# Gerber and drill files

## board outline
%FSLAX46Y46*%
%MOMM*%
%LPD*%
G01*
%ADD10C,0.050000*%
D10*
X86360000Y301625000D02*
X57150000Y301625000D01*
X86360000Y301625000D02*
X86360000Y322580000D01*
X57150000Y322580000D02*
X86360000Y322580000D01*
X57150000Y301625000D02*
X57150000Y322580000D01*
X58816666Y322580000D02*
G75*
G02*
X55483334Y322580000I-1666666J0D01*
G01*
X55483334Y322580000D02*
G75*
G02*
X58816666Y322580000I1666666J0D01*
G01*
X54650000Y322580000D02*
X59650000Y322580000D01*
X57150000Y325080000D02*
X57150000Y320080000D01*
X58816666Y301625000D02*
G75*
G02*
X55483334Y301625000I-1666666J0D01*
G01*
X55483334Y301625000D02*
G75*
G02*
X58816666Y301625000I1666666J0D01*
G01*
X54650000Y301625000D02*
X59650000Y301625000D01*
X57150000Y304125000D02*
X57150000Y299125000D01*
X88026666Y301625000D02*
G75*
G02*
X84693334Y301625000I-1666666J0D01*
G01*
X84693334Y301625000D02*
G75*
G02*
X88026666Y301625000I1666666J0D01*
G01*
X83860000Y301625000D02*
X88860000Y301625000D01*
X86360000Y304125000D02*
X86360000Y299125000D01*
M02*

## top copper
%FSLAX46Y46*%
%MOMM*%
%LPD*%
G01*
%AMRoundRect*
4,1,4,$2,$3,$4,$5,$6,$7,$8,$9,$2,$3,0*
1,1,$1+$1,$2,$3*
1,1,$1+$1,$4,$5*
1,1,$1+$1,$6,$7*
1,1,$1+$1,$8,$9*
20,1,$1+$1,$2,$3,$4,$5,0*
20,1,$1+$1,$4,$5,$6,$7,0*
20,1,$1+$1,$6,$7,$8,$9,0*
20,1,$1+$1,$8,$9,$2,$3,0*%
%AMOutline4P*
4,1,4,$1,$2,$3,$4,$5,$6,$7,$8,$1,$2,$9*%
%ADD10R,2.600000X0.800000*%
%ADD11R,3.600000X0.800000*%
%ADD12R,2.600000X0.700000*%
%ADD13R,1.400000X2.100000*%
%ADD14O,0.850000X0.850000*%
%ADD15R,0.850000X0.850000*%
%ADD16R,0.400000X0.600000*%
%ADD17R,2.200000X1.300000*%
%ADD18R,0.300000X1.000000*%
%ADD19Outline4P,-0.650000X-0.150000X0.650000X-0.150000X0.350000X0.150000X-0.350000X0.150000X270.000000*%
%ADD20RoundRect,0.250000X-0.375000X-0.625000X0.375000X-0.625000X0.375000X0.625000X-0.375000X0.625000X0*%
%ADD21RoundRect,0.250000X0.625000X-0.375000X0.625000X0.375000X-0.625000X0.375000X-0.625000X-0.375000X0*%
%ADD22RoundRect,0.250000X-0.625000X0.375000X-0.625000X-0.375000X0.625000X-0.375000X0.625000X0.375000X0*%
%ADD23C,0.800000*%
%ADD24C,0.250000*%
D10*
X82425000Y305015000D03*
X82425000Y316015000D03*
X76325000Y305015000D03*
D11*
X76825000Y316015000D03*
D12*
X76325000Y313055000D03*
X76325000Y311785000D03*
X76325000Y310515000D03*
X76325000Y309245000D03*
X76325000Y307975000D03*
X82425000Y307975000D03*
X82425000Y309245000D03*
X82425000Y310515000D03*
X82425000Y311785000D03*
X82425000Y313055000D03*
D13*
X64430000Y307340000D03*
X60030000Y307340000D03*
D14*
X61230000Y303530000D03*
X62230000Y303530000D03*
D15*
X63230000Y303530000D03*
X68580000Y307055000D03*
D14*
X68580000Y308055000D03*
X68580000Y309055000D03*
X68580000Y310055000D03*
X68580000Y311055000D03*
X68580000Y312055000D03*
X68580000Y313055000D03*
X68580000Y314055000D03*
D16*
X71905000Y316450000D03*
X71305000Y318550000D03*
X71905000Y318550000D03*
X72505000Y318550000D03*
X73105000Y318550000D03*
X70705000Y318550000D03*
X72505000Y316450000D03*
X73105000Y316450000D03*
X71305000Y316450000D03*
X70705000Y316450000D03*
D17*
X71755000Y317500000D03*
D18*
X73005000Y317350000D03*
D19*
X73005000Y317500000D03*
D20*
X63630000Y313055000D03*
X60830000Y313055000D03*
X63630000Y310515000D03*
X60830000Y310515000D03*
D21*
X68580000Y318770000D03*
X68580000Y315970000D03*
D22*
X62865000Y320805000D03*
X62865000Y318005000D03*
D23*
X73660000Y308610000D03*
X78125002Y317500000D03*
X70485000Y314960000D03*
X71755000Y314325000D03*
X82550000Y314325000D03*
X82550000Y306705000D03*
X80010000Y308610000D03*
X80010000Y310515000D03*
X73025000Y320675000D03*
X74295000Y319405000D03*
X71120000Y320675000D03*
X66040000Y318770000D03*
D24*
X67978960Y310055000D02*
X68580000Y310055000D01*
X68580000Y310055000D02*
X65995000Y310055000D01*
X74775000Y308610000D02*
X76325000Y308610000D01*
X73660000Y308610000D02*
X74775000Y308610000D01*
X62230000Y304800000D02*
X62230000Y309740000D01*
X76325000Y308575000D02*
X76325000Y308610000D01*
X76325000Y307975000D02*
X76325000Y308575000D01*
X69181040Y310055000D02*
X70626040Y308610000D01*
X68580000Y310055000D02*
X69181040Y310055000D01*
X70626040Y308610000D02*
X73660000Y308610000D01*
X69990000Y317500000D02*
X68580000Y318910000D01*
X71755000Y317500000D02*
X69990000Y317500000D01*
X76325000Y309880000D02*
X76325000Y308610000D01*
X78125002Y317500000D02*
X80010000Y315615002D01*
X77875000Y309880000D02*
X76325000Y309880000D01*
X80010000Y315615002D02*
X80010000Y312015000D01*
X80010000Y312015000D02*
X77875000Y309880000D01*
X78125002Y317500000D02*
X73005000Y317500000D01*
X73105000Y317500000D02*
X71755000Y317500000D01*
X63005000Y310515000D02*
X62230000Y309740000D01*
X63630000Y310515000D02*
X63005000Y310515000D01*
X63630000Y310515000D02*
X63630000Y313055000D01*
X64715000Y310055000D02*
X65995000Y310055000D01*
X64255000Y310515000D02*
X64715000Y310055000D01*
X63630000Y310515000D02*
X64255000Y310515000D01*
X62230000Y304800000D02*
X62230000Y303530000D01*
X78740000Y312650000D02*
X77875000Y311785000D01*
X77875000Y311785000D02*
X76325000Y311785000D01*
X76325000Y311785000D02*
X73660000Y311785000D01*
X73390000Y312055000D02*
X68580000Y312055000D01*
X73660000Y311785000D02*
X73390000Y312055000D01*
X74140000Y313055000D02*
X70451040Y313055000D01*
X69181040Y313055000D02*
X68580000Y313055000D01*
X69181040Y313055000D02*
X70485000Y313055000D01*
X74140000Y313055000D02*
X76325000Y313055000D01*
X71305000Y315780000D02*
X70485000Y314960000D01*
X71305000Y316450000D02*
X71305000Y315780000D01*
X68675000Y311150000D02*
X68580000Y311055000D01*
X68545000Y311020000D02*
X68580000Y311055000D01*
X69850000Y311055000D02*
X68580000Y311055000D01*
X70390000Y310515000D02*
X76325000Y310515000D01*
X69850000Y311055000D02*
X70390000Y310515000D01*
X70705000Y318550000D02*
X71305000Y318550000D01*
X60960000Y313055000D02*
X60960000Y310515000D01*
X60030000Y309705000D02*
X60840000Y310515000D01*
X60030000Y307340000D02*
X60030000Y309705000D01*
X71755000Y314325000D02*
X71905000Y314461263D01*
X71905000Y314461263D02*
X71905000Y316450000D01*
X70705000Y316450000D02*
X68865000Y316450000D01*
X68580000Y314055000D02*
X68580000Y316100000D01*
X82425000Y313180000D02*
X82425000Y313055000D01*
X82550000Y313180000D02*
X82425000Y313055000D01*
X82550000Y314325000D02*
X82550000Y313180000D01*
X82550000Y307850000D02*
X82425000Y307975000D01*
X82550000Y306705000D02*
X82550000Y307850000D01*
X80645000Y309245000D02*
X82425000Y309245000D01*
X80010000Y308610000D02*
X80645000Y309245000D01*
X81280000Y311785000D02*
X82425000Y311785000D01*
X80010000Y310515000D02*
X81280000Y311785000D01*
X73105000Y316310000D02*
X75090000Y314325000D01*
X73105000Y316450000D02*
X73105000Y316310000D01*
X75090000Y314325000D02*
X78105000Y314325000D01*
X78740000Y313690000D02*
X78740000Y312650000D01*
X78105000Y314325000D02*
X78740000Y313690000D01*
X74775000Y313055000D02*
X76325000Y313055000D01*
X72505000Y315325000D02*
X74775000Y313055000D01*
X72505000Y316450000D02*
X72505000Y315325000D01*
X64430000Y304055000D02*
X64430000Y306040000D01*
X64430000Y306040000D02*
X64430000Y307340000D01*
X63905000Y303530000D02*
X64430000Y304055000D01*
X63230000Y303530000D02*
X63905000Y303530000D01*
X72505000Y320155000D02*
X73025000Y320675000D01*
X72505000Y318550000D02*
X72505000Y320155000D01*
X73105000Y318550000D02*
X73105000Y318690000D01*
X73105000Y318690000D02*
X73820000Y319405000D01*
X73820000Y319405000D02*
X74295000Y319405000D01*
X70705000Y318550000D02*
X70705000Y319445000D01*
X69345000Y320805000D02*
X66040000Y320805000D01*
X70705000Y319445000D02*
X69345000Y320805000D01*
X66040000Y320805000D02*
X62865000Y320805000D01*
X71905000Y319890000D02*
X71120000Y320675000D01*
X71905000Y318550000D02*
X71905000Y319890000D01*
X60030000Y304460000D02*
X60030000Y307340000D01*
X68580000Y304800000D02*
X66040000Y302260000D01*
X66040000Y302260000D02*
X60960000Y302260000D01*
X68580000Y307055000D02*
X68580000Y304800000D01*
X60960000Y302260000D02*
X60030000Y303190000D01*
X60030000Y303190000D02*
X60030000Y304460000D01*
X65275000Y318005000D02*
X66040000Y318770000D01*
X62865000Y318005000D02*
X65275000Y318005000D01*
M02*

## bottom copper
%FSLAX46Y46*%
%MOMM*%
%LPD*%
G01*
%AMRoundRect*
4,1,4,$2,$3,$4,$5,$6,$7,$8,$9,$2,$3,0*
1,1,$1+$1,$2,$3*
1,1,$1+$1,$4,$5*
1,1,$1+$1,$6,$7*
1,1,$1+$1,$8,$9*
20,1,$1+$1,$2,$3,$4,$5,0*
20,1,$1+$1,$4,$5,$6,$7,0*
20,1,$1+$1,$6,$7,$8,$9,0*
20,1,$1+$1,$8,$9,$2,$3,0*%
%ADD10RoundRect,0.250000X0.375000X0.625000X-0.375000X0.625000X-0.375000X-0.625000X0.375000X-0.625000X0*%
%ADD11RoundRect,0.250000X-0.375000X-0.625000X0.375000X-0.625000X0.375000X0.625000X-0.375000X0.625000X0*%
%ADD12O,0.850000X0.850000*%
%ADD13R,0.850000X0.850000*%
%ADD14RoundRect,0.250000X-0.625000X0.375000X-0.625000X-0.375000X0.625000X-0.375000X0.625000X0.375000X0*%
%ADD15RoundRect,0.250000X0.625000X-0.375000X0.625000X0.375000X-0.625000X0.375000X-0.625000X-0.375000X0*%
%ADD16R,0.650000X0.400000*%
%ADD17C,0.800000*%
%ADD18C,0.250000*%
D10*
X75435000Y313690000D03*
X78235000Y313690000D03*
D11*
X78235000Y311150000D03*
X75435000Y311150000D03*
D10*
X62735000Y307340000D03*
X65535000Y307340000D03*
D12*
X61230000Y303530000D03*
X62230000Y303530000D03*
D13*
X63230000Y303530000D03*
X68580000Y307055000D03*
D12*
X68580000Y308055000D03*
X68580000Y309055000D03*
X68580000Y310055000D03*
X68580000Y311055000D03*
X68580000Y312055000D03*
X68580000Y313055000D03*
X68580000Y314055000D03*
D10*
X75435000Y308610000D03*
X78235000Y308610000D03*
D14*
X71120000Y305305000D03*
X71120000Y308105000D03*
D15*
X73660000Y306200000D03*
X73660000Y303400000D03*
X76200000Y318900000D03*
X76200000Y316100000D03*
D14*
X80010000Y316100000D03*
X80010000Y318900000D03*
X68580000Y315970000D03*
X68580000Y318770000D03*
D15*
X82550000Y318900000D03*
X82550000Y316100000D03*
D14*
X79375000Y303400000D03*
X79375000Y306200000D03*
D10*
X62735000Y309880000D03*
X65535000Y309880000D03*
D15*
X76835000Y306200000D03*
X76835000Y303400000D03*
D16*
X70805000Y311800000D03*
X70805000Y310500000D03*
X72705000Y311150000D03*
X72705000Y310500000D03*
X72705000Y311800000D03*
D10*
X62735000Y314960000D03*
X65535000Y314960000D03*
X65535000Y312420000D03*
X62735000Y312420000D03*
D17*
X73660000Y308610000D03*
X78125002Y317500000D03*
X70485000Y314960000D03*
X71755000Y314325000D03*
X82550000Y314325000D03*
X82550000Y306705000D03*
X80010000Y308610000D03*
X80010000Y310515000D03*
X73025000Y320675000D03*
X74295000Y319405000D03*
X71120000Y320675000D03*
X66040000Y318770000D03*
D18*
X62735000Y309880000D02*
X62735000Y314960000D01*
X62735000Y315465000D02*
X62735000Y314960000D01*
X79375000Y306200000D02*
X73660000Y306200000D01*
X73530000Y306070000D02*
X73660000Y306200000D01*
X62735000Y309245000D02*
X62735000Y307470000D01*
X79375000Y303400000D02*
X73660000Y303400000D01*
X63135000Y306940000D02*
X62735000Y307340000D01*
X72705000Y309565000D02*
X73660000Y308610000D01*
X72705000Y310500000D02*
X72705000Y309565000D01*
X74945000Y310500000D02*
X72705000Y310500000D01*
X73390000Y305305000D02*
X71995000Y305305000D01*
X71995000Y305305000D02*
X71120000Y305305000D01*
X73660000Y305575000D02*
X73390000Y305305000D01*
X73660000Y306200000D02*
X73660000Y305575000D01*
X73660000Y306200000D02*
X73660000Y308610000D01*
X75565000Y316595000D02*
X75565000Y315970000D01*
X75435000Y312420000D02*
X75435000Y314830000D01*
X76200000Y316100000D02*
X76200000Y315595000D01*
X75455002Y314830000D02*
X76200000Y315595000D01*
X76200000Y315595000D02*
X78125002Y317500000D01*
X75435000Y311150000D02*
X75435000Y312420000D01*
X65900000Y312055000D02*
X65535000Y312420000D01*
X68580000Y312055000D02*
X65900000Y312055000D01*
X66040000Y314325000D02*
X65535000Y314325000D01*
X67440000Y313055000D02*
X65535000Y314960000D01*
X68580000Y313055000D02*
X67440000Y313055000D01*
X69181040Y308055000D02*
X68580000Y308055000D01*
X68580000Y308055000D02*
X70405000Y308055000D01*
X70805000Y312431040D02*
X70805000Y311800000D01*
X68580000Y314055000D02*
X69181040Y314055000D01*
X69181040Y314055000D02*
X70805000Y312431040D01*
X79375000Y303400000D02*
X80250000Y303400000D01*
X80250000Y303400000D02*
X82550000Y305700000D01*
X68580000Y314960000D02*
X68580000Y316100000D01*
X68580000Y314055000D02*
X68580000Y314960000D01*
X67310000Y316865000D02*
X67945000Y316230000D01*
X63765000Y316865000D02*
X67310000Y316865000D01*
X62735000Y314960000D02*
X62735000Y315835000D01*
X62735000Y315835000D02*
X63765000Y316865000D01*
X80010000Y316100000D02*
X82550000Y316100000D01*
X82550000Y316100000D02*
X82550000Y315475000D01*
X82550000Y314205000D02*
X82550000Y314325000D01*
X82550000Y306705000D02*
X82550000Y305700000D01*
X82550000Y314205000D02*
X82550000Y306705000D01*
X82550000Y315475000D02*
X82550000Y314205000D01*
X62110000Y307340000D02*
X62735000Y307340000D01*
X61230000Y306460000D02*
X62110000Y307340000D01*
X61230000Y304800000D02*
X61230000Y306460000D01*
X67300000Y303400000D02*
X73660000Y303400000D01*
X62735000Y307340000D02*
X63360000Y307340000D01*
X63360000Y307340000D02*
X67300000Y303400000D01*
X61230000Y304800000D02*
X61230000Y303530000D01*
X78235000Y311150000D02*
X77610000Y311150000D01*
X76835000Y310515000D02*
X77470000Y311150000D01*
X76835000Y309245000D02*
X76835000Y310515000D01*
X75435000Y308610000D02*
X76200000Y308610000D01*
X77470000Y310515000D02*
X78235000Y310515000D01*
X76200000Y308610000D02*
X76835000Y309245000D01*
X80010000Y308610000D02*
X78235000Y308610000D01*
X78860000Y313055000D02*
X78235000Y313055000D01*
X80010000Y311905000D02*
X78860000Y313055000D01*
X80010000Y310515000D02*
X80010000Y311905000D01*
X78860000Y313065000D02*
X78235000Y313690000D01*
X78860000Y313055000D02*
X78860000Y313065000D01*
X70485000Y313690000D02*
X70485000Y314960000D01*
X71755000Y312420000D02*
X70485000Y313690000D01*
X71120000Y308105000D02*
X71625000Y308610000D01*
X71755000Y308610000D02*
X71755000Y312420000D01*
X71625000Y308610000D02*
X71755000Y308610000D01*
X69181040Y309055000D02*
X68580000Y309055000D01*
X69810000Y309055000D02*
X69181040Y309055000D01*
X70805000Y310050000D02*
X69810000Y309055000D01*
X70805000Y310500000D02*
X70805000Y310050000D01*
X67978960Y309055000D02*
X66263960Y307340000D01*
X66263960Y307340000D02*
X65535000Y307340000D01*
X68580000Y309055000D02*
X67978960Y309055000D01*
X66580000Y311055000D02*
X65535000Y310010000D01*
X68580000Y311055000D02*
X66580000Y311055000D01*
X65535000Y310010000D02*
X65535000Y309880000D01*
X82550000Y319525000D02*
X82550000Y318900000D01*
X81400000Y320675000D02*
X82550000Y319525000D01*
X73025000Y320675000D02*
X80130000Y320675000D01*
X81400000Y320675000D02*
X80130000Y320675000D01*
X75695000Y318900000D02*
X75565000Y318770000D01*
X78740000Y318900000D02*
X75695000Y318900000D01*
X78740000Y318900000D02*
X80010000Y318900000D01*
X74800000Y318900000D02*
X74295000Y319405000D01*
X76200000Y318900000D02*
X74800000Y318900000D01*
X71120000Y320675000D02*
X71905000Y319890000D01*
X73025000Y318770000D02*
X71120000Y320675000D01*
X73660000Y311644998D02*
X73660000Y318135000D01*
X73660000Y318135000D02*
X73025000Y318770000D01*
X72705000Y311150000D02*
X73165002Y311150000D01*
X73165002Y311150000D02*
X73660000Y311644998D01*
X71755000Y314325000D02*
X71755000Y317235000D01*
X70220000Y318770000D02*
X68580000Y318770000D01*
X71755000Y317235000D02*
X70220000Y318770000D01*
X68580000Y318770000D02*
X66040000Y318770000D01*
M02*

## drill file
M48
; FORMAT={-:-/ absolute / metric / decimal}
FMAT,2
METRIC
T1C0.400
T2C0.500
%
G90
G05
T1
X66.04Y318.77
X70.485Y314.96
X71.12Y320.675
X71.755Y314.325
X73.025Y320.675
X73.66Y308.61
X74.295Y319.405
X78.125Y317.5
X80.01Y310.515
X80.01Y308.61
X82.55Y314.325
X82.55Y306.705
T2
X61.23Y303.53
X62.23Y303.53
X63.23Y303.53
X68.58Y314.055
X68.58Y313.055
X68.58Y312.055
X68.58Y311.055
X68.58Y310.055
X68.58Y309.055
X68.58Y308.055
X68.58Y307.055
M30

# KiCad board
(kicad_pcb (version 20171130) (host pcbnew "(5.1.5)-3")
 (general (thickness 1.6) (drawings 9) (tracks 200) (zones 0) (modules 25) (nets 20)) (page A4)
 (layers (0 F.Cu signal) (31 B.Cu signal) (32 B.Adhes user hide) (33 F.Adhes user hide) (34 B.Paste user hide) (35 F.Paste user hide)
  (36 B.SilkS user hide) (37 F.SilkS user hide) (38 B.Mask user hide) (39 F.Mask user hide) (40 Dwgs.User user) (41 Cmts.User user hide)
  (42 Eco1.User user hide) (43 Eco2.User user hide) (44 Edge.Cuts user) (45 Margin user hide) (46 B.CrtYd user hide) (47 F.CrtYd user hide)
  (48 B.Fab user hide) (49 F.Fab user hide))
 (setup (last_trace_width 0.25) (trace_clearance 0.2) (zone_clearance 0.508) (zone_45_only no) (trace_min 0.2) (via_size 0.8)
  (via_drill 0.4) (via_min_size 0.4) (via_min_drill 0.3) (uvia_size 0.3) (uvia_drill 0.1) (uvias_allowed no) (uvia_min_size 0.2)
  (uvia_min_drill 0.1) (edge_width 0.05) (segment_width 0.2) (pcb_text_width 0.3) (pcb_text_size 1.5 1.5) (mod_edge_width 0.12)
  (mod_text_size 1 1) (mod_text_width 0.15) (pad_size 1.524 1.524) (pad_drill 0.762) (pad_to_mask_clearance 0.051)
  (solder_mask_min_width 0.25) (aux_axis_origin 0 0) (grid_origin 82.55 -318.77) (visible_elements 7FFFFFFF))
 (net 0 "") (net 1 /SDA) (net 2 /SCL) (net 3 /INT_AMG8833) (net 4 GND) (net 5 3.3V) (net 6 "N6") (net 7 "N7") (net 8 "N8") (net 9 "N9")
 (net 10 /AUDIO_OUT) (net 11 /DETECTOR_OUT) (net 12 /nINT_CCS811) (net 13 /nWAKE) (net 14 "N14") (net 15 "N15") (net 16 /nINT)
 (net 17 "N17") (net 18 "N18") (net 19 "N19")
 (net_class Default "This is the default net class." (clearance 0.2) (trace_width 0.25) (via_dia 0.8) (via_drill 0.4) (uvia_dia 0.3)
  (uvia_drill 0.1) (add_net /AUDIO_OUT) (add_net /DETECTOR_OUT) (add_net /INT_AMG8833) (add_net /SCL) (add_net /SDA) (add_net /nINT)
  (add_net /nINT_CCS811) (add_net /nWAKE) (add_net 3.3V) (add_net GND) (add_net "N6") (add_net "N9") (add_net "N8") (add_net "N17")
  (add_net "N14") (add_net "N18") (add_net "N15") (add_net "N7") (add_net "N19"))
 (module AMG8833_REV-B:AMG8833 (layer F.Cu) (at 79.375 -310.515 270)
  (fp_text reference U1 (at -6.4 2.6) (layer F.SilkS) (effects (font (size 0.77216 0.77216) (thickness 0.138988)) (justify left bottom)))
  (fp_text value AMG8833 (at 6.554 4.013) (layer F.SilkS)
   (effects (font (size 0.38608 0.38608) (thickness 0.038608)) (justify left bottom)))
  (pad 8 smd rect (at 5.5 -3.05) (size 2.6 0.8) (layers F.Cu F.Paste F.Mask) (solder_mask_margin 0.0508))
  (pad 14 smd rect (at -5.5 -3.05) (size 2.6 0.8) (layers F.Cu F.Paste F.Mask) (solder_mask_margin 0.0508))
  (pad 7 smd rect (at 5.5 3.05) (size 2.6 0.8) (layers F.Cu F.Paste F.Mask) (solder_mask_margin 0.0508))
  (pad 1 smd rect (at -5.5 2.55) (size 3.6 0.8) (layers F.Cu F.Paste F.Mask) (solder_mask_margin 0.0508))
  (pad 2 smd rect (at -2.54 3.05) (size 2.6 0.7) (layers F.Cu F.Paste F.Mask) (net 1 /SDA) (solder_mask_margin 0.0508))
  (pad 3 smd rect (at -1.27 3.05) (size 2.6 0.7) (layers F.Cu F.Paste F.Mask) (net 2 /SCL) (solder_mask_margin 0.0508))
  (pad 4 smd rect (at 0 3.05) (size 2.6 0.7) (layers F.Cu F.Paste F.Mask) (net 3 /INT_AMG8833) (solder_mask_margin 0.0508))
  (pad 5 smd rect (at 1.27 3.05) (size 2.6 0.7) (layers F.Cu F.Paste F.Mask) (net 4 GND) (solder_mask_margin 0.0508))
  (pad 6 smd rect (at 2.54 3.05) (size 2.6 0.7) (layers F.Cu F.Paste F.Mask) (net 4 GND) (solder_mask_margin 0.0508))
  (pad 9 smd rect (at 2.54 -3.05) (size 2.6 0.7) (layers F.Cu F.Paste F.Mask) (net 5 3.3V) (solder_mask_margin 0.0508))
  (pad 10 smd rect (at 1.27 -3.05) (size 2.6 0.7) (layers F.Cu F.Paste F.Mask) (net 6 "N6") (solder_mask_margin 0.0508))
  (pad 11 smd rect (at 0 -3.05) (size 2.6 0.7) (layers F.Cu F.Paste F.Mask) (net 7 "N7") (solder_mask_margin 0.0508))
  (pad 12 smd rect (at -1.27 -3.05) (size 2.6 0.7) (layers F.Cu F.Paste F.Mask) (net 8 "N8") (solder_mask_margin 0.0508))
  (pad 13 smd rect (at -2.54 -3.05) (size 2.6 0.7) (layers F.Cu F.Paste F.Mask) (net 5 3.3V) (solder_mask_margin 0.0508)))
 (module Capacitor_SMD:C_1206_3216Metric (layer B.Cu) (at 76.835 -313.69 180)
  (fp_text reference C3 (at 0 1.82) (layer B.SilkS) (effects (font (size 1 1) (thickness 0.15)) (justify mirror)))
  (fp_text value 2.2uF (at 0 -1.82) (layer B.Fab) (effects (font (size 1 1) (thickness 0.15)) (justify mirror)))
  (pad 2 smd roundrect (at 1.4 0 180) (size 1.25 1.75) (layers B.Cu B.Paste B.Mask) (roundrect_rratio 0.2) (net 4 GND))
  (pad 1 smd roundrect (at -1.4 0 180) (size 1.25 1.75) (layers B.Cu B.Paste B.Mask) (roundrect_rratio 0.2) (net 8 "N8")))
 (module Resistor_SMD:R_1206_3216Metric (layer B.Cu) (at 76.835 -311.15)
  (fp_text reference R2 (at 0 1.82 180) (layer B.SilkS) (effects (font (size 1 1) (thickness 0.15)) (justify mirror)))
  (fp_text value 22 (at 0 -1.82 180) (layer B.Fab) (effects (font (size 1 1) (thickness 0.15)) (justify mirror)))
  (pad 2 smd roundrect (at 1.4 0) (size 1.25 1.75) (layers B.Cu B.Paste B.Mask) (roundrect_rratio 0.2) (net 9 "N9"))
  (pad 1 smd roundrect (at -1.4 0) (size 1.25 1.75) (layers B.Cu B.Paste B.Mask) (roundrect_rratio 0.2) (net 4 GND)))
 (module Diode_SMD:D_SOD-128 (layer F.Cu) (at 62.23 -307.34)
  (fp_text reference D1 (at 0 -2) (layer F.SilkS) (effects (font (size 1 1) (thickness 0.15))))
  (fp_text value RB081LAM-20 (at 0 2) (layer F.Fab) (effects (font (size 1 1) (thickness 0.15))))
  (pad 2 smd rect (at 2.2 0) (size 1.4 2.1) (layers F.Cu F.Paste F.Mask) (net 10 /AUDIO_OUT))
  (pad 1 smd rect (at -2.2 0) (size 1.4 2.1) (layers F.Cu F.Paste F.Mask) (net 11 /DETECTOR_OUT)))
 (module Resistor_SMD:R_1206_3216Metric (layer B.Cu) (at 64.135 -307.34 180)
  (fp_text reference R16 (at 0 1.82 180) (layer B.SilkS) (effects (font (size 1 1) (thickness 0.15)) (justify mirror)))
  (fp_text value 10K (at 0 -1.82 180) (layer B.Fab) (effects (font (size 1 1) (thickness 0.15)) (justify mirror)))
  (pad 2 smd roundrect (at 1.4 0 180) (size 1.25 1.75) (layers B.Cu B.Paste B.Mask) (roundrect_rratio 0.2) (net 5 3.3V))
  (pad 1 smd roundrect (at -1.4 0 180) (size 1.25 1.75) (layers B.Cu B.Paste B.Mask) (roundrect_rratio 0.2) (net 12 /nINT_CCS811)))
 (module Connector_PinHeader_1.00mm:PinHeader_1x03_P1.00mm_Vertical (layer F.Cu) (at 63.23 -303.53 270)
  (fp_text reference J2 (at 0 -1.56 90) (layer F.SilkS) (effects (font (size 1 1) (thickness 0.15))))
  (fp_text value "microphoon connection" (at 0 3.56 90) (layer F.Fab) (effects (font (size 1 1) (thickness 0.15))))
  (pad 3 thru_hole oval (at 0 2 270) (size 0.85 0.85) (drill 0.5) (layers *.Cu *.Mask) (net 5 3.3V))
  (pad 2 thru_hole oval (at 0 1 270) (size 0.85 0.85) (drill 0.5) (layers *.Cu *.Mask) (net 4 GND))
  (pad 1 thru_hole rect (at 0 0 270) (size 0.85 0.85) (drill 0.5) (layers *.Cu *.Mask) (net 10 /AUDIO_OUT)))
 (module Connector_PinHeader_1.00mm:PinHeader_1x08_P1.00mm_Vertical (layer F.Cu) (at 68.58 -307.055 180)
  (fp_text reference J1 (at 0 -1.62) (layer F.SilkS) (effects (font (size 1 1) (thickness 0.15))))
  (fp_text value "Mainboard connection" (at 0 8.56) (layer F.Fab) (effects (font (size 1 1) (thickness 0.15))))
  (pad 1 thru_hole rect (at 0 0 180) (size 0.85 0.85) (drill 0.5) (layers *.Cu *.Mask) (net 11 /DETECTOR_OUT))
  (pad 2 thru_hole oval (at 0 1 180) (size 0.85 0.85) (drill 0.5) (layers *.Cu *.Mask) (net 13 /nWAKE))
  (pad 3 thru_hole oval (at 0 2 180) (size 0.85 0.85) (drill 0.5) (layers *.Cu *.Mask) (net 12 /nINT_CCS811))
  (pad 4 thru_hole oval (at 0 3 180) (size 0.85 0.85) (drill 0.5) (layers *.Cu *.Mask) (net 4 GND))
  (pad 5 thru_hole oval (at 0 4 180) (size 0.85 0.85) (drill 0.5) (layers *.Cu *.Mask) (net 3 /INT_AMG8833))
  (pad 6 thru_hole oval (at 0 5 180) (size 0.85 0.85) (drill 0.5) (layers *.Cu *.Mask) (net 2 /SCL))
  (pad 7 thru_hole oval (at 0 6 180) (size 0.85 0.85) (drill 0.5) (layers *.Cu *.Mask) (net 1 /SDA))
  (pad 8 thru_hole oval (at 0 7 180) (size 0.85 0.85) (drill 0.5) (layers *.Cu *.Mask) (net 5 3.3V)))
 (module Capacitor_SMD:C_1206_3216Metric (layer B.Cu) (at 76.835 -308.61 180)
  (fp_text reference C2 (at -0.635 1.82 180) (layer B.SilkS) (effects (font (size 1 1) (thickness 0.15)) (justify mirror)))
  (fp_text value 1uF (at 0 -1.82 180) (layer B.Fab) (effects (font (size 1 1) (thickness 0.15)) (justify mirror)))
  (pad 2 smd roundrect (at 1.4 0 180) (size 1.25 1.75) (layers B.Cu B.Paste B.Mask) (roundrect_rratio 0.2) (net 9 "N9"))
  (pad 1 smd roundrect (at -1.4 0 180) (size 1.25 1.75) (layers B.Cu B.Paste B.Mask) (roundrect_rratio 0.2) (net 6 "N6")))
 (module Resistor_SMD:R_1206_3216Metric (layer B.Cu) (at 71.12 -306.705 270)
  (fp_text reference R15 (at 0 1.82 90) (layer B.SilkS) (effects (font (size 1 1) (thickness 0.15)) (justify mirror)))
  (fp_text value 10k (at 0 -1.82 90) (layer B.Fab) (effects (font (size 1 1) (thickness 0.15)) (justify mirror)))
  (pad 2 smd roundrect (at 1.4 0 270) (size 1.25 1.75) (layers B.Cu B.Paste B.Mask) (roundrect_rratio 0.2) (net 4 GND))
  (pad 1 smd roundrect (at -1.4 0 270) (size 1.25 1.75) (layers B.Cu B.Paste B.Mask) (roundrect_rratio 0.2) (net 13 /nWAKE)))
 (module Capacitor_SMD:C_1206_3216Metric (layer B.Cu) (at 73.66 -304.8 90)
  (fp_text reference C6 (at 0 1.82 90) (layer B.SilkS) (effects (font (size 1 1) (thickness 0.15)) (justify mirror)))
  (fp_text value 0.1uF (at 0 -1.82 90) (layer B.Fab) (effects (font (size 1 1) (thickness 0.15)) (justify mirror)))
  (pad 2 smd roundrect (at 1.4 0 90) (size 1.25 1.75) (layers B.Cu B.Paste B.Mask) (roundrect_rratio 0.2) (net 4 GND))
  (pad 1 smd roundrect (at -1.4 0 90) (size 1.25 1.75) (layers B.Cu B.Paste B.Mask) (roundrect_rratio 0.2) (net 5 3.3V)))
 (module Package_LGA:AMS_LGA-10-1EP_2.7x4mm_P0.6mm (layer F.Cu) (at 71.905 -317.5 270)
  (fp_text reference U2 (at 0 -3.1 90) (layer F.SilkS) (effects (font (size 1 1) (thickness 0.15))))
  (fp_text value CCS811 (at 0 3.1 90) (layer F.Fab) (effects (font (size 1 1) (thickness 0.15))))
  (pad 8 smd rect (at 1.05 0 270) (size 0.6 0.4) (layers F.Cu F.Paste F.Mask) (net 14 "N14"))
  (pad 4 smd rect (at -1.05 0.6 270) (size 0.6 0.4) (layers F.Cu F.Paste F.Mask) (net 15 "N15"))
  (pad 3 smd rect (at -1.05 0 270) (size 0.6 0.4) (layers F.Cu F.Paste F.Mask) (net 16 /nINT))
  (pad 2 smd rect (at -1.05 -0.6 270) (size 0.6 0.4) (layers F.Cu F.Paste F.Mask) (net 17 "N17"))
  (pad 1 smd rect (at -1.05 -1.2 270) (size 0.6 0.4) (layers F.Cu F.Paste F.Mask) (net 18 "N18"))
  (pad 5 smd rect (at -1.05 1.2 270) (size 0.6 0.4) (layers F.Cu F.Paste F.Mask) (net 15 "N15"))
  (pad 9 smd rect (at 1.05 -0.6 270) (size 0.6 0.4) (layers F.Cu F.Paste F.Mask) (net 1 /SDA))
  (pad 10 smd rect (at 1.05 -1.2 270) (size 0.6 0.4) (layers F.Cu F.Paste F.Mask) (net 2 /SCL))
  (pad 7 smd rect (at 1.05 0.6 270) (size 0.6 0.4) (layers F.Cu F.Paste F.Mask) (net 13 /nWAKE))
  (pad 6 smd rect (at 1.05 1.2 270) (size 0.6 0.4) (layers F.Cu F.Paste F.Mask) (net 5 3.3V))
  (pad 11 smd rect (at 0 0.15 270) (size 1.3 2.2) (layers F.Cu F.Paste F.Mask) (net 4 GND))
  (pad 11 smd rect (at 0.15 -1.1 270) (size 1 0.3) (layers F.Cu F.Paste F.Mask) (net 4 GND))
  (pad 11 smd trapezoid (at 0 -1.1 270) (size 1 0.3) (rect_delta 0 0.3) (layers F.Cu F.Paste F.Mask) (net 4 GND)))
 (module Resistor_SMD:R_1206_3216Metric (layer F.Cu) (at 62.23 -313.055)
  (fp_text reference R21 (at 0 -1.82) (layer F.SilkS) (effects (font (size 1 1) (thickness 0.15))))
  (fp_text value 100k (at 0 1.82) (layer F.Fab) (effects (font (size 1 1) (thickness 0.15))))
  (pad 2 smd roundrect (at 1.4 0) (size 1.25 1.75) (layers F.Cu F.Paste F.Mask) (roundrect_rratio 0.2) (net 4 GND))
  (pad 1 smd roundrect (at -1.4 0) (size 1.25 1.75) (layers F.Cu F.Paste F.Mask) (roundrect_rratio 0.2) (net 11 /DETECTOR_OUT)))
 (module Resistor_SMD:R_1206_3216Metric (layer B.Cu) (at 76.2 -317.5 90)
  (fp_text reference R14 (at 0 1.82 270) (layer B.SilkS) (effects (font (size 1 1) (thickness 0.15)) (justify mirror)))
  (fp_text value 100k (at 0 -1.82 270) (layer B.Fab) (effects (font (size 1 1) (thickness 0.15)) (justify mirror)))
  (pad 2 smd roundrect (at 1.4 0 90) (size 1.25 1.75) (layers B.Cu B.Paste B.Mask) (roundrect_rratio 0.2) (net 18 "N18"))
  (pad 1 smd roundrect (at -1.4 0 90) (size 1.25 1.75) (layers B.Cu B.Paste B.Mask) (roundrect_rratio 0.2) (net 4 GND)))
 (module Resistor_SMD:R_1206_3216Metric (layer B.Cu) (at 80.01 -317.5 270)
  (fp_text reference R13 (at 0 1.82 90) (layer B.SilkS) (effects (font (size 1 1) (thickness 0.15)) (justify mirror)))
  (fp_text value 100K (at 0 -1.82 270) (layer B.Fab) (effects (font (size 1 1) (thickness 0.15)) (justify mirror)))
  (pad 2 smd roundrect (at 1.4 0 270) (size 1.25 1.75) (layers B.Cu B.Paste B.Mask) (roundrect_rratio 0.2) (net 5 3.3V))
  (pad 1 smd roundrect (at -1.4 0 270) (size 1.25 1.75) (layers B.Cu B.Paste B.Mask) (roundrect_rratio 0.2) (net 18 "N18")))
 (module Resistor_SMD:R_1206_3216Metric (layer B.Cu) (at 68.58 -317.37 270)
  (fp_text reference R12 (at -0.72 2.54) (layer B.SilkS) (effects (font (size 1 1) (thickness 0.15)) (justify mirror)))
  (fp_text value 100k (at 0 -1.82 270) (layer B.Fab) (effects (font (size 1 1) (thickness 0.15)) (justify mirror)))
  (pad 2 smd roundrect (at 1.4 0 270) (size 1.25 1.75) (layers B.Cu B.Paste B.Mask) (roundrect_rratio 0.2) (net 5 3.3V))
  (pad 1 smd roundrect (at -1.4 0 270) (size 1.25 1.75) (layers B.Cu B.Paste B.Mask) (roundrect_rratio 0.2) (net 14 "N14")))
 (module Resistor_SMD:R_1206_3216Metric (layer B.Cu) (at 82.55 -317.5 90)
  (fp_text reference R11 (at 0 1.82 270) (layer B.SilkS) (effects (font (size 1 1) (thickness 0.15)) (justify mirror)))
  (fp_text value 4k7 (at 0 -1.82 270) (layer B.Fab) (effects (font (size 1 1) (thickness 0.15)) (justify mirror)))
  (pad 2 smd roundrect (at 1.4 0 90) (size 1.25 1.75) (layers B.Cu B.Paste B.Mask) (roundrect_rratio 0.2) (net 17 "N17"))
  (pad 1 smd roundrect (at -1.4 0 90) (size 1.25 1.75) (layers B.Cu B.Paste B.Mask) (roundrect_rratio 0.2) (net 5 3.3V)))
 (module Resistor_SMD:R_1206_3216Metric (layer B.Cu) (at 79.375 -304.8 270)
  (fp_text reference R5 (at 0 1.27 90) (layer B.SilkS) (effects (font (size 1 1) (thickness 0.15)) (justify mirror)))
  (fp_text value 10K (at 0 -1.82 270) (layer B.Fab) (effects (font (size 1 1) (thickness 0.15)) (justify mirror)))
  (pad 2 smd roundrect (at 1.4 0 270) (size 1.25 1.75) (layers B.Cu B.Paste B.Mask) (roundrect_rratio 0.2) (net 5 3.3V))
  (pad 1 smd roundrect (at -1.4 0 270) (size 1.25 1.75) (layers B.Cu B.Paste B.Mask) (roundrect_rratio 0.2) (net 4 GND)))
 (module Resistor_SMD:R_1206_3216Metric (layer B.Cu) (at 64.135 -309.88 180)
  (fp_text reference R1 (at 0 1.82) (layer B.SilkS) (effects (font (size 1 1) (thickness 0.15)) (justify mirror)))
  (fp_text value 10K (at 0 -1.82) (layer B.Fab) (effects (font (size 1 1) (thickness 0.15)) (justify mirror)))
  (pad 2 smd roundrect (at 1.4 0 180) (size 1.25 1.75) (layers B.Cu B.Paste B.Mask) (roundrect_rratio 0.2) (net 5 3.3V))
  (pad 1 smd roundrect (at -1.4 0 180) (size 1.25 1.75) (layers B.Cu B.Paste B.Mask) (roundrect_rratio 0.2) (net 3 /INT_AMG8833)))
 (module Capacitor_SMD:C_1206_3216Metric (layer F.Cu) (at 62.23 -310.515)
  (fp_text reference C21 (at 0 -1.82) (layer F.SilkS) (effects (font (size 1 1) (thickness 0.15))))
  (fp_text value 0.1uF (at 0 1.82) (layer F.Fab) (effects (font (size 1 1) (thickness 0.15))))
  (pad 2 smd roundrect (at 1.4 0) (size 1.25 1.75) (layers F.Cu F.Paste F.Mask) (roundrect_rratio 0.2) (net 4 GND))
  (pad 1 smd roundrect (at -1.4 0) (size 1.25 1.75) (layers F.Cu F.Paste F.Mask) (roundrect_rratio 0.2) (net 11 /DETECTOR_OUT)))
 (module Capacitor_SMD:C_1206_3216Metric (layer F.Cu) (at 68.58 -317.37 90)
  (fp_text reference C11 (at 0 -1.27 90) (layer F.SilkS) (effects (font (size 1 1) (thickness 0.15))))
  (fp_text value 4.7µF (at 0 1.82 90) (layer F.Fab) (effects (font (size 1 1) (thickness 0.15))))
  (pad 2 smd roundrect (at 1.4 0 90) (size 1.25 1.75) (layers F.Cu F.Paste F.Mask) (roundrect_rratio 0.2) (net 4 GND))
  (pad 1 smd roundrect (at -1.4 0 90) (size 1.25 1.75) (layers F.Cu F.Paste F.Mask) (roundrect_rratio 0.2) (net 5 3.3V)))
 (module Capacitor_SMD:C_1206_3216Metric (layer B.Cu) (at 76.835 -304.8 90)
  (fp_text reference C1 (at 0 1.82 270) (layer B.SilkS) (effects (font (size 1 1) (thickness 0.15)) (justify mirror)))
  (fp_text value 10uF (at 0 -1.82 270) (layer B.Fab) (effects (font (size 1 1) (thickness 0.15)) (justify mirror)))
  (pad 2 smd roundrect (at 1.4 0 90) (size 1.25 1.75) (layers B.Cu B.Paste B.Mask) (roundrect_rratio 0.2) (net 4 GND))
  (pad 1 smd roundrect (at -1.4 0 90) (size 1.25 1.75) (layers B.Cu B.Paste B.Mask) (roundrect_rratio 0.2) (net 5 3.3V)))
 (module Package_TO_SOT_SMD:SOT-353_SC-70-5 (layer B.Cu) (at 71.755 -311.15 180)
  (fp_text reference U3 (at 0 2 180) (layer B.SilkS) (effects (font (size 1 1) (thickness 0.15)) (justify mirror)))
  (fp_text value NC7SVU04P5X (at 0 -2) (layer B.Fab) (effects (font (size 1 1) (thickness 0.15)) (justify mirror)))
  (pad 5 smd rect (at 0.95 0.65 180) (size 0.65 0.4) (layers B.Cu B.Paste B.Mask) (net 5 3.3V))
  (pad 4 smd rect (at 0.95 -0.65 180) (size 0.65 0.4) (layers B.Cu B.Paste B.Mask) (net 12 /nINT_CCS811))
  (pad 2 smd rect (at -0.95 0 180) (size 0.65 0.4) (layers B.Cu B.Paste B.Mask) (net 16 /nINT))
  (pad 3 smd rect (at -0.95 -0.65 180) (size 0.65 0.4) (layers B.Cu B.Paste B.Mask) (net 4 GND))
  (pad 1 smd rect (at -0.95 0.65 180) (size 0.65 0.4) (layers B.Cu B.Paste B.Mask) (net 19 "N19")))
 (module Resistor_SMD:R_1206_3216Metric (layer B.Cu) (at 64.135 -314.96 180)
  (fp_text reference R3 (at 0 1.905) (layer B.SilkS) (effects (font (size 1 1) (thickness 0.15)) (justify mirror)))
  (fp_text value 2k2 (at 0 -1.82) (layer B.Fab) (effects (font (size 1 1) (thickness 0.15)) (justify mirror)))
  (pad 2 smd roundrect (at 1.4 0 180) (size 1.25 1.75) (layers B.Cu B.Paste B.Mask) (roundrect_rratio 0.2) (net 5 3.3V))
  (pad 1 smd roundrect (at -1.4 0 180) (size 1.25 1.75) (layers B.Cu B.Paste B.Mask) (roundrect_rratio 0.2) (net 1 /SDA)))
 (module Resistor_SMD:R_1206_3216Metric (layer B.Cu) (at 64.135 -312.42 180)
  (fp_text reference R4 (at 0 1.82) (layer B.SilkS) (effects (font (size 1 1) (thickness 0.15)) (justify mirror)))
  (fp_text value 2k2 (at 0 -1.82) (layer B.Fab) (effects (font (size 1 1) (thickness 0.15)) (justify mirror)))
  (pad 1 smd roundrect (at -1.4 0 180) (size 1.25 1.75) (layers B.Cu B.Paste B.Mask) (roundrect_rratio 0.2) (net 2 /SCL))
  (pad 2 smd roundrect (at 1.4 0 180) (size 1.25 1.75) (layers B.Cu B.Paste B.Mask) (roundrect_rratio 0.2) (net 5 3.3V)))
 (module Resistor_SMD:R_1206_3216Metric (layer F.Cu) (at 62.865 -319.405 270)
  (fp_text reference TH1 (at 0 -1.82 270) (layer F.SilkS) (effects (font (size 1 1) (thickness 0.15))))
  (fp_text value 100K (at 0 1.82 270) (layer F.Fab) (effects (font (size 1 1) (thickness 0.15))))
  (pad 1 smd roundrect (at -1.4 0 270) (size 1.25 1.75) (layers F.Cu F.Paste F.Mask) (roundrect_rratio 0.2) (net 15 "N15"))
  (pad 2 smd roundrect (at 1.4 0 270) (size 1.25 1.75) (layers F.Cu F.Paste F.Mask) (roundrect_rratio 0.2) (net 14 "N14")))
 (gr_line (start 86.36 -301.625) (end 57.15 -301.625) (layer Edge.Cuts) (width 0.05))
 (gr_line (start 86.36 -301.625) (end 86.36 -322.58) (layer Edge.Cuts) (width 0.05))
 (gr_line (start 57.15 -322.58) (end 86.36 -322.58) (layer Edge.Cuts) (width 0.05))
 (gr_line (start 57.15 -301.625) (end 57.15 -322.58) (layer Edge.Cuts) (width 0.05))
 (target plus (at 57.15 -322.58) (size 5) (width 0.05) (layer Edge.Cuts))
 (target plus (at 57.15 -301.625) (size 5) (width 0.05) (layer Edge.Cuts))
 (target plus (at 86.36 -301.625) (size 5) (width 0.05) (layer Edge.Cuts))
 (segment (start 67.97896 -310.055) (end 68.58 -310.055) (width 0.25) (layer F.Cu) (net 4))
 (segment (start 62.735 -309.88) (end 62.735 -314.96) (width 0.25) (layer B.Cu) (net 5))
 (segment (start 62.735 -315.465) (end 62.735 -314.96) (width 0.25) (layer B.Cu) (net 5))
 (segment (start 79.375 -306.2) (end 73.66 -306.2) (width 0.25) (layer B.Cu) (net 4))
 (segment (start 68.58 -310.055) (end 65.995 -310.055) (width 0.25) (layer F.Cu) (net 4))
 (segment (start 74.775 -308.61) (end 76.325 -308.61) (width 0.25) (layer F.Cu) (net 4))
 (segment (start 73.66 -308.61) (end 74.775 -308.61) (width 0.25) (layer F.Cu) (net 4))
 (via (at 73.66 -308.61) (size 0.8) (drill 0.4) (layers F.Cu B.Cu) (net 4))
 (segment (start 73.53 -306.07) (end 73.66 -306.2) (width 0.25) (layer B.Cu) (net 4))
 (segment (start 62.23 -304.8) (end 62.23 -309.74) (width 0.25) (layer F.Cu) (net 4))
 (segment (start 76.325 -308.575) (end 76.325 -308.61) (width 0.25) (layer F.Cu) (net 4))
 (segment (start 76.325 -307.975) (end 76.325 -308.575) (width 0.25) (layer F.Cu) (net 4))
 (segment (start 69.18104 -310.055) (end 70.62604 -308.61) (width 0.25) (layer F.Cu) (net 4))
 (segment (start 68.58 -310.055) (end 69.18104 -310.055) (width 0.25) (layer F.Cu) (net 4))
 (segment (start 70.62604 -308.61) (end 73.66 -308.61) (width 0.25) (layer F.Cu) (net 4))
 (segment (start 69.99 -317.5) (end 68.58 -318.91) (width 0.25) (layer F.Cu) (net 4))
 (segment (start 71.755 -317.5) (end 69.99 -317.5) (width 0.25) (layer F.Cu) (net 4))
 (segment (start 62.735 -309.245) (end 62.735 -307.47) (width 0.25) (layer B.Cu) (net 5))
 (segment (start 79.375 -303.4) (end 73.66 -303.4) (width 0.25) (layer B.Cu) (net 5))
 (segment (start 63.135 -306.94) (end 62.735 -307.34) (width 0.25) (layer B.Cu) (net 5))
 (segment (start 72.705 -309.565) (end 73.66 -308.61) (width 0.25) (layer B.Cu) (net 4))
 (segment (start 72.705 -310.5) (end 72.705 -309.565) (width 0.25) (layer B.Cu) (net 4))
 (segment (start 74.945 -310.5) (end 72.705 -310.5) (width 0.25) (layer B.Cu) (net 4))
 (segment (start 73.39 -305.305) (end 71.995 -305.305) (width 0.25) (layer B.Cu) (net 4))
 (segment (start 71.995 -305.305) (end 71.12 -305.305) (width 0.25) (layer B.Cu) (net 4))
 (segment (start 73.66 -305.575) (end 73.39 -305.305) (width 0.25) (layer B.Cu) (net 4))
 (segment (start 73.66 -306.2) (end 73.66 -305.575) (width 0.25) (layer B.Cu) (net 4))
 (segment (start 73.66 -306.2) (end 73.66 -308.61) (width 0.25) (layer B.Cu) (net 4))
 (segment (start 76.325 -309.88) (end 76.325 -308.61) (width 0.25) (layer F.Cu) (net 4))
 (segment (start 78.125002 -317.5) (end 80.01 -315.615002) (width 0.25) (layer F.Cu) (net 4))
 (segment (start 77.875 -309.88) (end 76.325 -309.88) (width 0.25) (layer F.Cu) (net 4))
 (segment (start 80.01 -315.615002) (end 80.01 -312.015) (width 0.25) (layer F.Cu) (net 4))
 (segment (start 80.01 -312.015) (end 77.875 -309.88) (width 0.25) (layer F.Cu) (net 4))
 (segment (start 78.125002 -317.5) (end 73.005 -317.5) (width 0.25) (layer F.Cu) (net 4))
 (via (at 78.125002 -317.5) (size 0.8) (drill 0.4) (layers F.Cu B.Cu) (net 4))
 (segment (start 75.565 -316.595) (end 75.565 -315.97) (width 0.25) (layer B.Cu) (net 4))
 (segment (start 73.105 -317.5) (end 71.755 -317.5) (width 0.25) (layer F.Cu) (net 4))
 (segment (start 75.435 -312.42) (end 75.435 -314.83) (width 0.25) (layer B.Cu) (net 4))
 (segment (start 76.2 -316.1) (end 76.2 -315.595) (width 0.25) (layer B.Cu) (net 4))
 (segment (start 75.455002 -314.83) (end 76.2 -315.595) (width 0.25) (layer B.Cu) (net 4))
 (segment (start 76.2 -315.595) (end 78.125002 -317.5) (width 0.25) (layer B.Cu) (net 4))
 (segment (start 75.435 -311.15) (end 75.435 -312.42) (width 0.25) (layer B.Cu) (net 4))
 (segment (start 63.005 -310.515) (end 62.23 -309.74) (width 0.25) (layer F.Cu) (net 4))
 (segment (start 63.63 -310.515) (end 63.005 -310.515) (width 0.25) (layer F.Cu) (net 4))
 (segment (start 63.63 -310.515) (end 63.63 -313.055) (width 0.25) (layer F.Cu) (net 4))
 (segment (start 64.715 -310.055) (end 65.995 -310.055) (width 0.25) (layer F.Cu) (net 4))
 (segment (start 64.255 -310.515) (end 64.715 -310.055) (width 0.25) (layer F.Cu) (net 4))
 (segment (start 63.63 -310.515) (end 64.255 -310.515) (width 0.25) (layer F.Cu) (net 4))
 (segment (start 62.23 -304.8) (end 62.23 -303.53) (width 0.25) (layer F.Cu) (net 4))
 (segment (start 65.9 -312.055) (end 65.535 -312.42) (width 0.25) (layer B.Cu) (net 2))
 (segment (start 68.58 -312.055) (end 65.9 -312.055) (width 0.25) (layer B.Cu) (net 2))
 (segment (start 78.74 -312.65) (end 77.875 -311.785) (width 0.25) (layer F.Cu) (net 2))
 (segment (start 77.875 -311.785) (end 76.325 -311.785) (width 0.25) (layer F.Cu) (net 2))
 (segment (start 76.325 -311.785) (end 73.66 -311.785) (width 0.25) (layer F.Cu) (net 2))
 (segment (start 73.39 -312.055) (end 68.58 -312.055) (width 0.25) (layer F.Cu) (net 2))
 (segment (start 73.66 -311.785) (end 73.39 -312.055) (width 0.25) (layer F.Cu) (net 2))
 (segment (start 74.14 -313.055) (end 70.45104 -313.055) (width 0.25) (layer F.Cu) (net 1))
 (segment (start 69.18104 -313.055) (end 68.58 -313.055) (width 0.25) (layer F.Cu) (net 1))
 (segment (start 69.18104 -313.055) (end 70.485 -313.055) (width 0.25) (layer F.Cu) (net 1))
 (segment (start 66.04 -314.325) (end 65.535 -314.325) (width 0.25) (layer B.Cu) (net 1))
 (segment (start 67.44 -313.055) (end 65.535 -314.96) (width 0.25) (layer B.Cu) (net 1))
 (segment (start 68.58 -313.055) (end 67.44 -313.055) (width 0.25) (layer B.Cu) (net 1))
 (segment (start 74.14 -313.055) (end 76.325 -313.055) (width 0.25) (layer F.Cu) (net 1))
 (via (at 70.485 -314.96) (size 0.8) (drill 0.4) (layers F.Cu B.Cu) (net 13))
 (segment (start 71.305 -315.78) (end 70.485 -314.96) (width 0.25) (layer F.Cu) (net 13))
 (segment (start 71.305 -316.45) (end 71.305 -315.78) (width 0.25) (layer F.Cu) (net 13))
 (segment (start 69.18104 -308.055) (end 68.58 -308.055) (width 0.25) (layer B.Cu) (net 13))
 (segment (start 68.58 -308.055) (end 70.405 -308.055) (width 0.25) (layer B.Cu) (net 13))
 (segment (start 68.675 -311.15) (end 68.58 -311.055) (width 0.25) (layer F.Cu) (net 3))
 (segment (start 68.545 -311.02) (end 68.58 -311.055) (width 0.25) (layer F.Cu) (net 3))
 (segment (start 69.85 -311.055) (end 68.58 -311.055) (width 0.25) (layer F.Cu) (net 3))
 (segment (start 70.39 -310.515) (end 76.325 -310.515) (width 0.25) (layer F.Cu) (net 3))
 (segment (start 69.85 -311.055) (end 70.39 -310.515) (width 0.25) (layer F.Cu) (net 3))
 (segment (start 70.705 -318.55) (end 71.305 -318.55) (width 0.25) (layer F.Cu) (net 15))
 (segment (start 60.96 -313.055) (end 60.96 -310.515) (width 0.25) (layer F.Cu) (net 11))
 (segment (start 60.03 -309.705) (end 60.84 -310.515) (width 0.25) (layer F.Cu) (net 11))
 (segment (start 60.03 -307.34) (end 60.03 -309.705) (width 0.25) (layer F.Cu) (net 11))
 (segment (start 71.755 -314.325) (end 71.905 -314.461263) (width 0.25) (layer F.Cu) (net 14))
 (via (at 71.755 -314.325) (size 0.8) (drill 0.4) (layers F.Cu B.Cu) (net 14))
 (segment (start 71.905 -314.461263) (end 71.905 -316.45) (width 0.25) (layer F.Cu) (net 14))
 (segment (start 70.705 -316.45) (end 68.865 -316.45) (width 0.25) (layer F.Cu) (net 5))
 (segment (start 68.58 -314.055) (end 68.58 -316.1) (width 0.25) (layer F.Cu) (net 5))
 (segment (start 70.805 -312.43104) (end 70.805 -311.8) (width 0.25) (layer B.Cu) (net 5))
 (segment (start 68.58 -314.055) (end 69.18104 -314.055) (width 0.25) (layer B.Cu) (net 5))
 (segment (start 69.18104 -314.055) (end 70.805 -312.43104) (width 0.25) (layer B.Cu) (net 5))
 (segment (start 79.375 -303.4) (end 80.25 -303.4) (width 0.25) (layer B.Cu) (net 5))
 (segment (start 80.25 -303.4) (end 82.55 -305.7) (width 0.25) (layer B.Cu) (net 5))
 (segment (start 68.58 -314.96) (end 68.58 -316.1) (width 0.25) (layer B.Cu) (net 5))
 (segment (start 68.58 -314.055) (end 68.58 -314.96) (width 0.25) (layer B.Cu) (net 5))
 (segment (start 67.31 -316.865) (end 67.945 -316.23) (width 0.25) (layer B.Cu) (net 5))
 (segment (start 63.765 -316.865) (end 67.31 -316.865) (width 0.25) (layer B.Cu) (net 5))
 (segment (start 62.735 -314.96) (end 62.735 -315.835) (width 0.25) (layer B.Cu) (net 5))
 (segment (start 62.735 -315.835) (end 63.765 -316.865) (width 0.25) (layer B.Cu) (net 5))
 (segment (start 82.425 -313.18) (end 82.425 -313.055) (width 0.25) (layer F.Cu) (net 5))
 (segment (start 80.01 -316.1) (end 82.55 -316.1) (width 0.25) (layer B.Cu) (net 5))
 (segment (start 82.55 -316.1) (end 82.55 -315.475) (width 0.25) (layer B.Cu) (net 5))
 (via (at 82.55 -314.325) (size 0.8) (drill 0.4) (layers F.Cu B.Cu) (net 5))
 (segment (start 82.55 -314.205) (end 82.55 -314.325) (width 0.25) (layer B.Cu) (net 5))
 (segment (start 82.55 -313.18) (end 82.425 -313.055) (width 0.25) (layer F.Cu) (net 5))
 (segment (start 82.55 -314.325) (end 82.55 -313.18) (width 0.25) (layer F.Cu) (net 5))
 (via (at 82.55 -306.705) (size 0.8) (drill 0.4) (layers F.Cu B.Cu) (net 5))
 (segment (start 82.55 -306.705) (end 82.55 -305.7) (width 0.25) (layer B.Cu) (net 5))
 (segment (start 82.55 -314.205) (end 82.55 -306.705) (width 0.25) (layer B.Cu) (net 5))
 (segment (start 82.55 -307.85) (end 82.425 -307.975) (width 0.25) (layer F.Cu) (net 5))
 (segment (start 82.55 -306.705) (end 82.55 -307.85) (width 0.25) (layer F.Cu) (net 5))
 (segment (start 82.55 -315.475) (end 82.55 -314.205) (width 0.25) (layer B.Cu) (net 5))
 (segment (start 62.11 -307.34) (end 62.735 -307.34) (width 0.25) (layer B.Cu) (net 5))
 (segment (start 61.23 -306.46) (end 62.11 -307.34) (width 0.25) (layer B.Cu) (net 5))
 (segment (start 61.23 -304.8) (end 61.23 -306.46) (width 0.25) (layer B.Cu) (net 5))
 (segment (start 67.3 -303.4) (end 73.66 -303.4) (width 0.25) (layer B.Cu) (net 5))
 (segment (start 62.735 -307.34) (end 63.36 -307.34) (width 0.25) (layer B.Cu) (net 5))
 (segment (start 63.36 -307.34) (end 67.3 -303.4) (width 0.25) (layer B.Cu) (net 5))
 (segment (start 61.23 -304.8) (end 61.23 -303.53) (width 0.25) (layer B.Cu) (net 5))
 (segment (start 78.235 -311.15) (end 77.61 -311.15) (width 0.25) (layer B.Cu) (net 9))
 (segment (start 76.835 -310.515) (end 77.47 -311.15) (width 0.25) (layer B.Cu) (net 9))
 (segment (start 76.835 -309.245) (end 76.835 -310.515) (width 0.25) (layer B.Cu) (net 9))
 (segment (start 75.435 -308.61) (end 76.2 -308.61) (width 0.25) (layer B.Cu) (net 9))
 (segment (start 77.47 -310.515) (end 78.235 -310.515) (width 0.25) (layer B.Cu) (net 9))
 (segment (start 76.2 -308.61) (end 76.835 -309.245) (width 0.25) (layer B.Cu) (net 9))
 (segment (start 80.645 -309.245) (end 82.425 -309.245) (width 0.25) (layer F.Cu) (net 6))
 (via (at 80.01 -308.61) (size 0.8) (drill 0.4) (layers F.Cu B.Cu) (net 6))
 (segment (start 80.01 -308.61) (end 80.645 -309.245) (width 0.25) (layer F.Cu) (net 6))
 (segment (start 80.01 -308.61) (end 78.235 -308.61) (width 0.25) (layer B.Cu) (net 6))
 (via (at 80.01 -310.515) (size 0.8) (drill 0.4) (layers F.Cu B.Cu) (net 8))
 (segment (start 81.28 -311.785) (end 82.425 -311.785) (width 0.25) (layer F.Cu) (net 8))
 (segment (start 80.01 -310.515) (end 81.28 -311.785) (width 0.25) (layer F.Cu) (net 8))
 (segment (start 78.86 -313.055) (end 78.235 -313.055) (width 0.25) (layer B.Cu) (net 8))
 (segment (start 80.01 -311.905) (end 78.86 -313.055) (width 0.25) (layer B.Cu) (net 8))
 (segment (start 80.01 -310.515) (end 80.01 -311.905) (width 0.25) (layer B.Cu) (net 8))
 (segment (start 78.86 -313.065) (end 78.235 -313.69) (width 0.25) (layer B.Cu) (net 8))
 (segment (start 78.86 -313.055) (end 78.86 -313.065) (width 0.25) (layer B.Cu) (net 8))
 (segment (start 73.105 -316.31) (end 75.09 -314.325) (width 0.25) (layer F.Cu) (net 2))
 (segment (start 73.105 -316.45) (end 73.105 -316.31) (width 0.25) (layer F.Cu) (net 2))
 (segment (start 75.09 -314.325) (end 78.105 -314.325) (width 0.25) (layer F.Cu) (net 2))
 (segment (start 78.74 -313.69) (end 78.74 -312.65) (width 0.25) (layer F.Cu) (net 2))
 (segment (start 78.105 -314.325) (end 78.74 -313.69) (width 0.25) (layer F.Cu) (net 2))
 (segment (start 74.775 -313.055) (end 76.325 -313.055) (width 0.25) (layer F.Cu) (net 1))
 (segment (start 72.505 -315.325) (end 74.775 -313.055) (width 0.25) (layer F.Cu) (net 1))
 (segment (start 72.505 -316.45) (end 72.505 -315.325) (width 0.25) (layer F.Cu) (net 1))
 (segment (start 64.43 -304.055) (end 64.43 -306.04) (width 0.25) (layer F.Cu) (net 10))
 (segment (start 64.43 -306.04) (end 64.43 -307.34) (width 0.25) (layer F.Cu) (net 10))
 (segment (start 63.905 -303.53) (end 64.43 -304.055) (width 0.25) (layer F.Cu) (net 10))
 (segment (start 63.23 -303.53) (end 63.905 -303.53) (width 0.25) (layer F.Cu) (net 10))
 (segment (start 70.485 -313.69) (end 70.485 -314.96) (width 0.25) (layer B.Cu) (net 13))
 (segment (start 71.755 -312.42) (end 70.485 -313.69) (width 0.25) (layer B.Cu) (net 13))
 (segment (start 71.12 -308.105) (end 71.625 -308.61) (width 0.25) (layer B.Cu) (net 13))
 (segment (start 71.755 -308.61) (end 71.755 -312.42) (width 0.25) (layer B.Cu) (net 13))
 (segment (start 71.625 -308.61) (end 71.755 -308.61) (width 0.25) (layer B.Cu) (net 13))
 (segment (start 69.18104 -309.055) (end 68.58 -309.055) (width 0.25) (layer B.Cu) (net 12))
 (segment (start 69.81 -309.055) (end 69.18104 -309.055) (width 0.25) (layer B.Cu) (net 12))
 (segment (start 70.805 -310.05) (end 69.81 -309.055) (width 0.25) (layer B.Cu) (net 12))
 (segment (start 70.805 -310.5) (end 70.805 -310.05) (width 0.25) (layer B.Cu) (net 12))
 (segment (start 67.97896 -309.055) (end 66.26396 -307.34) (width 0.25) (layer B.Cu) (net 12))
 (segment (start 66.26396 -307.34) (end 65.535 -307.34) (width 0.25) (layer B.Cu) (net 12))
 (segment (start 68.58 -309.055) (end 67.97896 -309.055) (width 0.25) (layer B.Cu) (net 12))
 (segment (start 66.58 -311.055) (end 65.535 -310.01) (width 0.25) (layer B.Cu) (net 3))
 (segment (start 68.58 -311.055) (end 66.58 -311.055) (width 0.25) (layer B.Cu) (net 3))
 (segment (start 65.535 -310.01) (end 65.535 -309.88) (width 0.25) (layer B.Cu) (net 3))
 (via (at 73.025 -320.675) (size 0.8) (drill 0.4) (layers F.Cu B.Cu) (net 17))
 (segment (start 72.505 -320.155) (end 73.025 -320.675) (width 0.25) (layer F.Cu) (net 17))
 (segment (start 72.505 -318.55) (end 72.505 -320.155) (width 0.25) (layer F.Cu) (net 17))
 (segment (start 82.55 -319.525) (end 82.55 -318.9) (width 0.25) (layer B.Cu) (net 17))
 (segment (start 81.4 -320.675) (end 82.55 -319.525) (width 0.25) (layer B.Cu) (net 17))
 (segment (start 73.025 -320.675) (end 80.13 -320.675) (width 0.25) (layer B.Cu) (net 17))
 (segment (start 81.4 -320.675) (end 80.13 -320.675) (width 0.25) (layer B.Cu) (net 17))
 (segment (start 75.695 -318.9) (end 75.565 -318.77) (width 0.25) (layer B.Cu) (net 18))
 (segment (start 78.74 -318.9) (end 75.695 -318.9) (width 0.25) (layer B.Cu) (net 18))
 (segment (start 78.74 -318.9) (end 80.01 -318.9) (width 0.25) (layer B.Cu) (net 18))
 (via (at 74.295 -319.405) (size 0.8) (drill 0.4) (layers F.Cu B.Cu) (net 18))
 (segment (start 73.105 -318.55) (end 73.105 -318.69) (width 0.25) (layer F.Cu) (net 18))
 (segment (start 73.105 -318.69) (end 73.82 -319.405) (width 0.25) (layer F.Cu) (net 18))
 (segment (start 73.82 -319.405) (end 74.295 -319.405) (width 0.25) (layer F.Cu) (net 18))
 (segment (start 74.8 -318.9) (end 74.295 -319.405) (width 0.25) (layer B.Cu) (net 18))
 (segment (start 76.2 -318.9) (end 74.8 -318.9) (width 0.25) (layer B.Cu) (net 18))
 (segment (start 70.705 -318.55) (end 70.705 -319.445) (width 0.25) (layer F.Cu) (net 15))
 (segment (start 69.345 -320.805) (end 66.04 -320.805) (width 0.25) (layer F.Cu) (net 15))
 (segment (start 70.705 -319.445) (end 69.345 -320.805) (width 0.25) (layer F.Cu) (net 15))
 (segment (start 66.04 -320.805) (end 62.865 -320.805) (width 0.25) (layer F.Cu) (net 15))
 (via (at 71.12 -320.675) (size 0.8) (drill 0.4) (layers F.Cu B.Cu) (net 16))
 (segment (start 71.905 -319.89) (end 71.12 -320.675) (width 0.25) (layer F.Cu) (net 16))
 (segment (start 71.905 -318.55) (end 71.905 -319.89) (width 0.25) (layer F.Cu) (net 16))
 (segment (start 71.12 -320.675) (end 71.905 -319.89) (width 0.25) (layer B.Cu) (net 16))
 (segment (start 73.025 -318.77) (end 71.12 -320.675) (width 0.25) (layer B.Cu) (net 16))
 (segment (start 73.66 -311.644998) (end 73.66 -318.135) (width 0.25) (layer B.Cu) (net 16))
 (segment (start 73.66 -318.135) (end 73.025 -318.77) (width 0.25) (layer B.Cu) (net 16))
 (segment (start 72.705 -311.15) (end 73.165002 -311.15) (width 0.25) (layer B.Cu) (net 16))
 (segment (start 73.165002 -311.15) (end 73.66 -311.644998) (width 0.25) (layer B.Cu) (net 16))
 (segment (start 60.03 -304.46) (end 60.03 -307.34) (width 0.25) (layer F.Cu) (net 11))
 (segment (start 68.58 -304.8) (end 66.04 -302.26) (width 0.25) (layer F.Cu) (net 11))
 (segment (start 66.04 -302.26) (end 60.96 -302.26) (width 0.25) (layer F.Cu) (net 11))
 (segment (start 68.58 -307.055) (end 68.58 -304.8) (width 0.25) (layer F.Cu) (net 11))
 (segment (start 60.96 -302.26) (end 60.03 -303.19) (width 0.25) (layer F.Cu) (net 11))
 (segment (start 60.03 -303.19) (end 60.03 -304.46) (width 0.25) (layer F.Cu) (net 11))
 (segment (start 71.755 -314.325) (end 71.755 -317.235) (width 0.25) (layer B.Cu) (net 14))
 (segment (start 70.22 -318.77) (end 68.58 -318.77) (width 0.25) (layer B.Cu) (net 14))
 (segment (start 71.755 -317.235) (end 70.22 -318.77) (width 0.25) (layer B.Cu) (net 14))
 (segment (start 68.58 -318.77) (end 66.04 -318.77) (width 0.25) (layer B.Cu) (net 14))
 (via (at 66.04 -318.77) (size 0.8) (drill 0.4) (layers F.Cu B.Cu) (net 14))
 (segment (start 65.275 -318.005) (end 66.04 -318.77) (width 0.25) (layer F.Cu) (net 14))
 (segment (start 62.865 -318.005) (end 65.275 -318.005) (width 0.25) (layer F.Cu) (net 14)))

